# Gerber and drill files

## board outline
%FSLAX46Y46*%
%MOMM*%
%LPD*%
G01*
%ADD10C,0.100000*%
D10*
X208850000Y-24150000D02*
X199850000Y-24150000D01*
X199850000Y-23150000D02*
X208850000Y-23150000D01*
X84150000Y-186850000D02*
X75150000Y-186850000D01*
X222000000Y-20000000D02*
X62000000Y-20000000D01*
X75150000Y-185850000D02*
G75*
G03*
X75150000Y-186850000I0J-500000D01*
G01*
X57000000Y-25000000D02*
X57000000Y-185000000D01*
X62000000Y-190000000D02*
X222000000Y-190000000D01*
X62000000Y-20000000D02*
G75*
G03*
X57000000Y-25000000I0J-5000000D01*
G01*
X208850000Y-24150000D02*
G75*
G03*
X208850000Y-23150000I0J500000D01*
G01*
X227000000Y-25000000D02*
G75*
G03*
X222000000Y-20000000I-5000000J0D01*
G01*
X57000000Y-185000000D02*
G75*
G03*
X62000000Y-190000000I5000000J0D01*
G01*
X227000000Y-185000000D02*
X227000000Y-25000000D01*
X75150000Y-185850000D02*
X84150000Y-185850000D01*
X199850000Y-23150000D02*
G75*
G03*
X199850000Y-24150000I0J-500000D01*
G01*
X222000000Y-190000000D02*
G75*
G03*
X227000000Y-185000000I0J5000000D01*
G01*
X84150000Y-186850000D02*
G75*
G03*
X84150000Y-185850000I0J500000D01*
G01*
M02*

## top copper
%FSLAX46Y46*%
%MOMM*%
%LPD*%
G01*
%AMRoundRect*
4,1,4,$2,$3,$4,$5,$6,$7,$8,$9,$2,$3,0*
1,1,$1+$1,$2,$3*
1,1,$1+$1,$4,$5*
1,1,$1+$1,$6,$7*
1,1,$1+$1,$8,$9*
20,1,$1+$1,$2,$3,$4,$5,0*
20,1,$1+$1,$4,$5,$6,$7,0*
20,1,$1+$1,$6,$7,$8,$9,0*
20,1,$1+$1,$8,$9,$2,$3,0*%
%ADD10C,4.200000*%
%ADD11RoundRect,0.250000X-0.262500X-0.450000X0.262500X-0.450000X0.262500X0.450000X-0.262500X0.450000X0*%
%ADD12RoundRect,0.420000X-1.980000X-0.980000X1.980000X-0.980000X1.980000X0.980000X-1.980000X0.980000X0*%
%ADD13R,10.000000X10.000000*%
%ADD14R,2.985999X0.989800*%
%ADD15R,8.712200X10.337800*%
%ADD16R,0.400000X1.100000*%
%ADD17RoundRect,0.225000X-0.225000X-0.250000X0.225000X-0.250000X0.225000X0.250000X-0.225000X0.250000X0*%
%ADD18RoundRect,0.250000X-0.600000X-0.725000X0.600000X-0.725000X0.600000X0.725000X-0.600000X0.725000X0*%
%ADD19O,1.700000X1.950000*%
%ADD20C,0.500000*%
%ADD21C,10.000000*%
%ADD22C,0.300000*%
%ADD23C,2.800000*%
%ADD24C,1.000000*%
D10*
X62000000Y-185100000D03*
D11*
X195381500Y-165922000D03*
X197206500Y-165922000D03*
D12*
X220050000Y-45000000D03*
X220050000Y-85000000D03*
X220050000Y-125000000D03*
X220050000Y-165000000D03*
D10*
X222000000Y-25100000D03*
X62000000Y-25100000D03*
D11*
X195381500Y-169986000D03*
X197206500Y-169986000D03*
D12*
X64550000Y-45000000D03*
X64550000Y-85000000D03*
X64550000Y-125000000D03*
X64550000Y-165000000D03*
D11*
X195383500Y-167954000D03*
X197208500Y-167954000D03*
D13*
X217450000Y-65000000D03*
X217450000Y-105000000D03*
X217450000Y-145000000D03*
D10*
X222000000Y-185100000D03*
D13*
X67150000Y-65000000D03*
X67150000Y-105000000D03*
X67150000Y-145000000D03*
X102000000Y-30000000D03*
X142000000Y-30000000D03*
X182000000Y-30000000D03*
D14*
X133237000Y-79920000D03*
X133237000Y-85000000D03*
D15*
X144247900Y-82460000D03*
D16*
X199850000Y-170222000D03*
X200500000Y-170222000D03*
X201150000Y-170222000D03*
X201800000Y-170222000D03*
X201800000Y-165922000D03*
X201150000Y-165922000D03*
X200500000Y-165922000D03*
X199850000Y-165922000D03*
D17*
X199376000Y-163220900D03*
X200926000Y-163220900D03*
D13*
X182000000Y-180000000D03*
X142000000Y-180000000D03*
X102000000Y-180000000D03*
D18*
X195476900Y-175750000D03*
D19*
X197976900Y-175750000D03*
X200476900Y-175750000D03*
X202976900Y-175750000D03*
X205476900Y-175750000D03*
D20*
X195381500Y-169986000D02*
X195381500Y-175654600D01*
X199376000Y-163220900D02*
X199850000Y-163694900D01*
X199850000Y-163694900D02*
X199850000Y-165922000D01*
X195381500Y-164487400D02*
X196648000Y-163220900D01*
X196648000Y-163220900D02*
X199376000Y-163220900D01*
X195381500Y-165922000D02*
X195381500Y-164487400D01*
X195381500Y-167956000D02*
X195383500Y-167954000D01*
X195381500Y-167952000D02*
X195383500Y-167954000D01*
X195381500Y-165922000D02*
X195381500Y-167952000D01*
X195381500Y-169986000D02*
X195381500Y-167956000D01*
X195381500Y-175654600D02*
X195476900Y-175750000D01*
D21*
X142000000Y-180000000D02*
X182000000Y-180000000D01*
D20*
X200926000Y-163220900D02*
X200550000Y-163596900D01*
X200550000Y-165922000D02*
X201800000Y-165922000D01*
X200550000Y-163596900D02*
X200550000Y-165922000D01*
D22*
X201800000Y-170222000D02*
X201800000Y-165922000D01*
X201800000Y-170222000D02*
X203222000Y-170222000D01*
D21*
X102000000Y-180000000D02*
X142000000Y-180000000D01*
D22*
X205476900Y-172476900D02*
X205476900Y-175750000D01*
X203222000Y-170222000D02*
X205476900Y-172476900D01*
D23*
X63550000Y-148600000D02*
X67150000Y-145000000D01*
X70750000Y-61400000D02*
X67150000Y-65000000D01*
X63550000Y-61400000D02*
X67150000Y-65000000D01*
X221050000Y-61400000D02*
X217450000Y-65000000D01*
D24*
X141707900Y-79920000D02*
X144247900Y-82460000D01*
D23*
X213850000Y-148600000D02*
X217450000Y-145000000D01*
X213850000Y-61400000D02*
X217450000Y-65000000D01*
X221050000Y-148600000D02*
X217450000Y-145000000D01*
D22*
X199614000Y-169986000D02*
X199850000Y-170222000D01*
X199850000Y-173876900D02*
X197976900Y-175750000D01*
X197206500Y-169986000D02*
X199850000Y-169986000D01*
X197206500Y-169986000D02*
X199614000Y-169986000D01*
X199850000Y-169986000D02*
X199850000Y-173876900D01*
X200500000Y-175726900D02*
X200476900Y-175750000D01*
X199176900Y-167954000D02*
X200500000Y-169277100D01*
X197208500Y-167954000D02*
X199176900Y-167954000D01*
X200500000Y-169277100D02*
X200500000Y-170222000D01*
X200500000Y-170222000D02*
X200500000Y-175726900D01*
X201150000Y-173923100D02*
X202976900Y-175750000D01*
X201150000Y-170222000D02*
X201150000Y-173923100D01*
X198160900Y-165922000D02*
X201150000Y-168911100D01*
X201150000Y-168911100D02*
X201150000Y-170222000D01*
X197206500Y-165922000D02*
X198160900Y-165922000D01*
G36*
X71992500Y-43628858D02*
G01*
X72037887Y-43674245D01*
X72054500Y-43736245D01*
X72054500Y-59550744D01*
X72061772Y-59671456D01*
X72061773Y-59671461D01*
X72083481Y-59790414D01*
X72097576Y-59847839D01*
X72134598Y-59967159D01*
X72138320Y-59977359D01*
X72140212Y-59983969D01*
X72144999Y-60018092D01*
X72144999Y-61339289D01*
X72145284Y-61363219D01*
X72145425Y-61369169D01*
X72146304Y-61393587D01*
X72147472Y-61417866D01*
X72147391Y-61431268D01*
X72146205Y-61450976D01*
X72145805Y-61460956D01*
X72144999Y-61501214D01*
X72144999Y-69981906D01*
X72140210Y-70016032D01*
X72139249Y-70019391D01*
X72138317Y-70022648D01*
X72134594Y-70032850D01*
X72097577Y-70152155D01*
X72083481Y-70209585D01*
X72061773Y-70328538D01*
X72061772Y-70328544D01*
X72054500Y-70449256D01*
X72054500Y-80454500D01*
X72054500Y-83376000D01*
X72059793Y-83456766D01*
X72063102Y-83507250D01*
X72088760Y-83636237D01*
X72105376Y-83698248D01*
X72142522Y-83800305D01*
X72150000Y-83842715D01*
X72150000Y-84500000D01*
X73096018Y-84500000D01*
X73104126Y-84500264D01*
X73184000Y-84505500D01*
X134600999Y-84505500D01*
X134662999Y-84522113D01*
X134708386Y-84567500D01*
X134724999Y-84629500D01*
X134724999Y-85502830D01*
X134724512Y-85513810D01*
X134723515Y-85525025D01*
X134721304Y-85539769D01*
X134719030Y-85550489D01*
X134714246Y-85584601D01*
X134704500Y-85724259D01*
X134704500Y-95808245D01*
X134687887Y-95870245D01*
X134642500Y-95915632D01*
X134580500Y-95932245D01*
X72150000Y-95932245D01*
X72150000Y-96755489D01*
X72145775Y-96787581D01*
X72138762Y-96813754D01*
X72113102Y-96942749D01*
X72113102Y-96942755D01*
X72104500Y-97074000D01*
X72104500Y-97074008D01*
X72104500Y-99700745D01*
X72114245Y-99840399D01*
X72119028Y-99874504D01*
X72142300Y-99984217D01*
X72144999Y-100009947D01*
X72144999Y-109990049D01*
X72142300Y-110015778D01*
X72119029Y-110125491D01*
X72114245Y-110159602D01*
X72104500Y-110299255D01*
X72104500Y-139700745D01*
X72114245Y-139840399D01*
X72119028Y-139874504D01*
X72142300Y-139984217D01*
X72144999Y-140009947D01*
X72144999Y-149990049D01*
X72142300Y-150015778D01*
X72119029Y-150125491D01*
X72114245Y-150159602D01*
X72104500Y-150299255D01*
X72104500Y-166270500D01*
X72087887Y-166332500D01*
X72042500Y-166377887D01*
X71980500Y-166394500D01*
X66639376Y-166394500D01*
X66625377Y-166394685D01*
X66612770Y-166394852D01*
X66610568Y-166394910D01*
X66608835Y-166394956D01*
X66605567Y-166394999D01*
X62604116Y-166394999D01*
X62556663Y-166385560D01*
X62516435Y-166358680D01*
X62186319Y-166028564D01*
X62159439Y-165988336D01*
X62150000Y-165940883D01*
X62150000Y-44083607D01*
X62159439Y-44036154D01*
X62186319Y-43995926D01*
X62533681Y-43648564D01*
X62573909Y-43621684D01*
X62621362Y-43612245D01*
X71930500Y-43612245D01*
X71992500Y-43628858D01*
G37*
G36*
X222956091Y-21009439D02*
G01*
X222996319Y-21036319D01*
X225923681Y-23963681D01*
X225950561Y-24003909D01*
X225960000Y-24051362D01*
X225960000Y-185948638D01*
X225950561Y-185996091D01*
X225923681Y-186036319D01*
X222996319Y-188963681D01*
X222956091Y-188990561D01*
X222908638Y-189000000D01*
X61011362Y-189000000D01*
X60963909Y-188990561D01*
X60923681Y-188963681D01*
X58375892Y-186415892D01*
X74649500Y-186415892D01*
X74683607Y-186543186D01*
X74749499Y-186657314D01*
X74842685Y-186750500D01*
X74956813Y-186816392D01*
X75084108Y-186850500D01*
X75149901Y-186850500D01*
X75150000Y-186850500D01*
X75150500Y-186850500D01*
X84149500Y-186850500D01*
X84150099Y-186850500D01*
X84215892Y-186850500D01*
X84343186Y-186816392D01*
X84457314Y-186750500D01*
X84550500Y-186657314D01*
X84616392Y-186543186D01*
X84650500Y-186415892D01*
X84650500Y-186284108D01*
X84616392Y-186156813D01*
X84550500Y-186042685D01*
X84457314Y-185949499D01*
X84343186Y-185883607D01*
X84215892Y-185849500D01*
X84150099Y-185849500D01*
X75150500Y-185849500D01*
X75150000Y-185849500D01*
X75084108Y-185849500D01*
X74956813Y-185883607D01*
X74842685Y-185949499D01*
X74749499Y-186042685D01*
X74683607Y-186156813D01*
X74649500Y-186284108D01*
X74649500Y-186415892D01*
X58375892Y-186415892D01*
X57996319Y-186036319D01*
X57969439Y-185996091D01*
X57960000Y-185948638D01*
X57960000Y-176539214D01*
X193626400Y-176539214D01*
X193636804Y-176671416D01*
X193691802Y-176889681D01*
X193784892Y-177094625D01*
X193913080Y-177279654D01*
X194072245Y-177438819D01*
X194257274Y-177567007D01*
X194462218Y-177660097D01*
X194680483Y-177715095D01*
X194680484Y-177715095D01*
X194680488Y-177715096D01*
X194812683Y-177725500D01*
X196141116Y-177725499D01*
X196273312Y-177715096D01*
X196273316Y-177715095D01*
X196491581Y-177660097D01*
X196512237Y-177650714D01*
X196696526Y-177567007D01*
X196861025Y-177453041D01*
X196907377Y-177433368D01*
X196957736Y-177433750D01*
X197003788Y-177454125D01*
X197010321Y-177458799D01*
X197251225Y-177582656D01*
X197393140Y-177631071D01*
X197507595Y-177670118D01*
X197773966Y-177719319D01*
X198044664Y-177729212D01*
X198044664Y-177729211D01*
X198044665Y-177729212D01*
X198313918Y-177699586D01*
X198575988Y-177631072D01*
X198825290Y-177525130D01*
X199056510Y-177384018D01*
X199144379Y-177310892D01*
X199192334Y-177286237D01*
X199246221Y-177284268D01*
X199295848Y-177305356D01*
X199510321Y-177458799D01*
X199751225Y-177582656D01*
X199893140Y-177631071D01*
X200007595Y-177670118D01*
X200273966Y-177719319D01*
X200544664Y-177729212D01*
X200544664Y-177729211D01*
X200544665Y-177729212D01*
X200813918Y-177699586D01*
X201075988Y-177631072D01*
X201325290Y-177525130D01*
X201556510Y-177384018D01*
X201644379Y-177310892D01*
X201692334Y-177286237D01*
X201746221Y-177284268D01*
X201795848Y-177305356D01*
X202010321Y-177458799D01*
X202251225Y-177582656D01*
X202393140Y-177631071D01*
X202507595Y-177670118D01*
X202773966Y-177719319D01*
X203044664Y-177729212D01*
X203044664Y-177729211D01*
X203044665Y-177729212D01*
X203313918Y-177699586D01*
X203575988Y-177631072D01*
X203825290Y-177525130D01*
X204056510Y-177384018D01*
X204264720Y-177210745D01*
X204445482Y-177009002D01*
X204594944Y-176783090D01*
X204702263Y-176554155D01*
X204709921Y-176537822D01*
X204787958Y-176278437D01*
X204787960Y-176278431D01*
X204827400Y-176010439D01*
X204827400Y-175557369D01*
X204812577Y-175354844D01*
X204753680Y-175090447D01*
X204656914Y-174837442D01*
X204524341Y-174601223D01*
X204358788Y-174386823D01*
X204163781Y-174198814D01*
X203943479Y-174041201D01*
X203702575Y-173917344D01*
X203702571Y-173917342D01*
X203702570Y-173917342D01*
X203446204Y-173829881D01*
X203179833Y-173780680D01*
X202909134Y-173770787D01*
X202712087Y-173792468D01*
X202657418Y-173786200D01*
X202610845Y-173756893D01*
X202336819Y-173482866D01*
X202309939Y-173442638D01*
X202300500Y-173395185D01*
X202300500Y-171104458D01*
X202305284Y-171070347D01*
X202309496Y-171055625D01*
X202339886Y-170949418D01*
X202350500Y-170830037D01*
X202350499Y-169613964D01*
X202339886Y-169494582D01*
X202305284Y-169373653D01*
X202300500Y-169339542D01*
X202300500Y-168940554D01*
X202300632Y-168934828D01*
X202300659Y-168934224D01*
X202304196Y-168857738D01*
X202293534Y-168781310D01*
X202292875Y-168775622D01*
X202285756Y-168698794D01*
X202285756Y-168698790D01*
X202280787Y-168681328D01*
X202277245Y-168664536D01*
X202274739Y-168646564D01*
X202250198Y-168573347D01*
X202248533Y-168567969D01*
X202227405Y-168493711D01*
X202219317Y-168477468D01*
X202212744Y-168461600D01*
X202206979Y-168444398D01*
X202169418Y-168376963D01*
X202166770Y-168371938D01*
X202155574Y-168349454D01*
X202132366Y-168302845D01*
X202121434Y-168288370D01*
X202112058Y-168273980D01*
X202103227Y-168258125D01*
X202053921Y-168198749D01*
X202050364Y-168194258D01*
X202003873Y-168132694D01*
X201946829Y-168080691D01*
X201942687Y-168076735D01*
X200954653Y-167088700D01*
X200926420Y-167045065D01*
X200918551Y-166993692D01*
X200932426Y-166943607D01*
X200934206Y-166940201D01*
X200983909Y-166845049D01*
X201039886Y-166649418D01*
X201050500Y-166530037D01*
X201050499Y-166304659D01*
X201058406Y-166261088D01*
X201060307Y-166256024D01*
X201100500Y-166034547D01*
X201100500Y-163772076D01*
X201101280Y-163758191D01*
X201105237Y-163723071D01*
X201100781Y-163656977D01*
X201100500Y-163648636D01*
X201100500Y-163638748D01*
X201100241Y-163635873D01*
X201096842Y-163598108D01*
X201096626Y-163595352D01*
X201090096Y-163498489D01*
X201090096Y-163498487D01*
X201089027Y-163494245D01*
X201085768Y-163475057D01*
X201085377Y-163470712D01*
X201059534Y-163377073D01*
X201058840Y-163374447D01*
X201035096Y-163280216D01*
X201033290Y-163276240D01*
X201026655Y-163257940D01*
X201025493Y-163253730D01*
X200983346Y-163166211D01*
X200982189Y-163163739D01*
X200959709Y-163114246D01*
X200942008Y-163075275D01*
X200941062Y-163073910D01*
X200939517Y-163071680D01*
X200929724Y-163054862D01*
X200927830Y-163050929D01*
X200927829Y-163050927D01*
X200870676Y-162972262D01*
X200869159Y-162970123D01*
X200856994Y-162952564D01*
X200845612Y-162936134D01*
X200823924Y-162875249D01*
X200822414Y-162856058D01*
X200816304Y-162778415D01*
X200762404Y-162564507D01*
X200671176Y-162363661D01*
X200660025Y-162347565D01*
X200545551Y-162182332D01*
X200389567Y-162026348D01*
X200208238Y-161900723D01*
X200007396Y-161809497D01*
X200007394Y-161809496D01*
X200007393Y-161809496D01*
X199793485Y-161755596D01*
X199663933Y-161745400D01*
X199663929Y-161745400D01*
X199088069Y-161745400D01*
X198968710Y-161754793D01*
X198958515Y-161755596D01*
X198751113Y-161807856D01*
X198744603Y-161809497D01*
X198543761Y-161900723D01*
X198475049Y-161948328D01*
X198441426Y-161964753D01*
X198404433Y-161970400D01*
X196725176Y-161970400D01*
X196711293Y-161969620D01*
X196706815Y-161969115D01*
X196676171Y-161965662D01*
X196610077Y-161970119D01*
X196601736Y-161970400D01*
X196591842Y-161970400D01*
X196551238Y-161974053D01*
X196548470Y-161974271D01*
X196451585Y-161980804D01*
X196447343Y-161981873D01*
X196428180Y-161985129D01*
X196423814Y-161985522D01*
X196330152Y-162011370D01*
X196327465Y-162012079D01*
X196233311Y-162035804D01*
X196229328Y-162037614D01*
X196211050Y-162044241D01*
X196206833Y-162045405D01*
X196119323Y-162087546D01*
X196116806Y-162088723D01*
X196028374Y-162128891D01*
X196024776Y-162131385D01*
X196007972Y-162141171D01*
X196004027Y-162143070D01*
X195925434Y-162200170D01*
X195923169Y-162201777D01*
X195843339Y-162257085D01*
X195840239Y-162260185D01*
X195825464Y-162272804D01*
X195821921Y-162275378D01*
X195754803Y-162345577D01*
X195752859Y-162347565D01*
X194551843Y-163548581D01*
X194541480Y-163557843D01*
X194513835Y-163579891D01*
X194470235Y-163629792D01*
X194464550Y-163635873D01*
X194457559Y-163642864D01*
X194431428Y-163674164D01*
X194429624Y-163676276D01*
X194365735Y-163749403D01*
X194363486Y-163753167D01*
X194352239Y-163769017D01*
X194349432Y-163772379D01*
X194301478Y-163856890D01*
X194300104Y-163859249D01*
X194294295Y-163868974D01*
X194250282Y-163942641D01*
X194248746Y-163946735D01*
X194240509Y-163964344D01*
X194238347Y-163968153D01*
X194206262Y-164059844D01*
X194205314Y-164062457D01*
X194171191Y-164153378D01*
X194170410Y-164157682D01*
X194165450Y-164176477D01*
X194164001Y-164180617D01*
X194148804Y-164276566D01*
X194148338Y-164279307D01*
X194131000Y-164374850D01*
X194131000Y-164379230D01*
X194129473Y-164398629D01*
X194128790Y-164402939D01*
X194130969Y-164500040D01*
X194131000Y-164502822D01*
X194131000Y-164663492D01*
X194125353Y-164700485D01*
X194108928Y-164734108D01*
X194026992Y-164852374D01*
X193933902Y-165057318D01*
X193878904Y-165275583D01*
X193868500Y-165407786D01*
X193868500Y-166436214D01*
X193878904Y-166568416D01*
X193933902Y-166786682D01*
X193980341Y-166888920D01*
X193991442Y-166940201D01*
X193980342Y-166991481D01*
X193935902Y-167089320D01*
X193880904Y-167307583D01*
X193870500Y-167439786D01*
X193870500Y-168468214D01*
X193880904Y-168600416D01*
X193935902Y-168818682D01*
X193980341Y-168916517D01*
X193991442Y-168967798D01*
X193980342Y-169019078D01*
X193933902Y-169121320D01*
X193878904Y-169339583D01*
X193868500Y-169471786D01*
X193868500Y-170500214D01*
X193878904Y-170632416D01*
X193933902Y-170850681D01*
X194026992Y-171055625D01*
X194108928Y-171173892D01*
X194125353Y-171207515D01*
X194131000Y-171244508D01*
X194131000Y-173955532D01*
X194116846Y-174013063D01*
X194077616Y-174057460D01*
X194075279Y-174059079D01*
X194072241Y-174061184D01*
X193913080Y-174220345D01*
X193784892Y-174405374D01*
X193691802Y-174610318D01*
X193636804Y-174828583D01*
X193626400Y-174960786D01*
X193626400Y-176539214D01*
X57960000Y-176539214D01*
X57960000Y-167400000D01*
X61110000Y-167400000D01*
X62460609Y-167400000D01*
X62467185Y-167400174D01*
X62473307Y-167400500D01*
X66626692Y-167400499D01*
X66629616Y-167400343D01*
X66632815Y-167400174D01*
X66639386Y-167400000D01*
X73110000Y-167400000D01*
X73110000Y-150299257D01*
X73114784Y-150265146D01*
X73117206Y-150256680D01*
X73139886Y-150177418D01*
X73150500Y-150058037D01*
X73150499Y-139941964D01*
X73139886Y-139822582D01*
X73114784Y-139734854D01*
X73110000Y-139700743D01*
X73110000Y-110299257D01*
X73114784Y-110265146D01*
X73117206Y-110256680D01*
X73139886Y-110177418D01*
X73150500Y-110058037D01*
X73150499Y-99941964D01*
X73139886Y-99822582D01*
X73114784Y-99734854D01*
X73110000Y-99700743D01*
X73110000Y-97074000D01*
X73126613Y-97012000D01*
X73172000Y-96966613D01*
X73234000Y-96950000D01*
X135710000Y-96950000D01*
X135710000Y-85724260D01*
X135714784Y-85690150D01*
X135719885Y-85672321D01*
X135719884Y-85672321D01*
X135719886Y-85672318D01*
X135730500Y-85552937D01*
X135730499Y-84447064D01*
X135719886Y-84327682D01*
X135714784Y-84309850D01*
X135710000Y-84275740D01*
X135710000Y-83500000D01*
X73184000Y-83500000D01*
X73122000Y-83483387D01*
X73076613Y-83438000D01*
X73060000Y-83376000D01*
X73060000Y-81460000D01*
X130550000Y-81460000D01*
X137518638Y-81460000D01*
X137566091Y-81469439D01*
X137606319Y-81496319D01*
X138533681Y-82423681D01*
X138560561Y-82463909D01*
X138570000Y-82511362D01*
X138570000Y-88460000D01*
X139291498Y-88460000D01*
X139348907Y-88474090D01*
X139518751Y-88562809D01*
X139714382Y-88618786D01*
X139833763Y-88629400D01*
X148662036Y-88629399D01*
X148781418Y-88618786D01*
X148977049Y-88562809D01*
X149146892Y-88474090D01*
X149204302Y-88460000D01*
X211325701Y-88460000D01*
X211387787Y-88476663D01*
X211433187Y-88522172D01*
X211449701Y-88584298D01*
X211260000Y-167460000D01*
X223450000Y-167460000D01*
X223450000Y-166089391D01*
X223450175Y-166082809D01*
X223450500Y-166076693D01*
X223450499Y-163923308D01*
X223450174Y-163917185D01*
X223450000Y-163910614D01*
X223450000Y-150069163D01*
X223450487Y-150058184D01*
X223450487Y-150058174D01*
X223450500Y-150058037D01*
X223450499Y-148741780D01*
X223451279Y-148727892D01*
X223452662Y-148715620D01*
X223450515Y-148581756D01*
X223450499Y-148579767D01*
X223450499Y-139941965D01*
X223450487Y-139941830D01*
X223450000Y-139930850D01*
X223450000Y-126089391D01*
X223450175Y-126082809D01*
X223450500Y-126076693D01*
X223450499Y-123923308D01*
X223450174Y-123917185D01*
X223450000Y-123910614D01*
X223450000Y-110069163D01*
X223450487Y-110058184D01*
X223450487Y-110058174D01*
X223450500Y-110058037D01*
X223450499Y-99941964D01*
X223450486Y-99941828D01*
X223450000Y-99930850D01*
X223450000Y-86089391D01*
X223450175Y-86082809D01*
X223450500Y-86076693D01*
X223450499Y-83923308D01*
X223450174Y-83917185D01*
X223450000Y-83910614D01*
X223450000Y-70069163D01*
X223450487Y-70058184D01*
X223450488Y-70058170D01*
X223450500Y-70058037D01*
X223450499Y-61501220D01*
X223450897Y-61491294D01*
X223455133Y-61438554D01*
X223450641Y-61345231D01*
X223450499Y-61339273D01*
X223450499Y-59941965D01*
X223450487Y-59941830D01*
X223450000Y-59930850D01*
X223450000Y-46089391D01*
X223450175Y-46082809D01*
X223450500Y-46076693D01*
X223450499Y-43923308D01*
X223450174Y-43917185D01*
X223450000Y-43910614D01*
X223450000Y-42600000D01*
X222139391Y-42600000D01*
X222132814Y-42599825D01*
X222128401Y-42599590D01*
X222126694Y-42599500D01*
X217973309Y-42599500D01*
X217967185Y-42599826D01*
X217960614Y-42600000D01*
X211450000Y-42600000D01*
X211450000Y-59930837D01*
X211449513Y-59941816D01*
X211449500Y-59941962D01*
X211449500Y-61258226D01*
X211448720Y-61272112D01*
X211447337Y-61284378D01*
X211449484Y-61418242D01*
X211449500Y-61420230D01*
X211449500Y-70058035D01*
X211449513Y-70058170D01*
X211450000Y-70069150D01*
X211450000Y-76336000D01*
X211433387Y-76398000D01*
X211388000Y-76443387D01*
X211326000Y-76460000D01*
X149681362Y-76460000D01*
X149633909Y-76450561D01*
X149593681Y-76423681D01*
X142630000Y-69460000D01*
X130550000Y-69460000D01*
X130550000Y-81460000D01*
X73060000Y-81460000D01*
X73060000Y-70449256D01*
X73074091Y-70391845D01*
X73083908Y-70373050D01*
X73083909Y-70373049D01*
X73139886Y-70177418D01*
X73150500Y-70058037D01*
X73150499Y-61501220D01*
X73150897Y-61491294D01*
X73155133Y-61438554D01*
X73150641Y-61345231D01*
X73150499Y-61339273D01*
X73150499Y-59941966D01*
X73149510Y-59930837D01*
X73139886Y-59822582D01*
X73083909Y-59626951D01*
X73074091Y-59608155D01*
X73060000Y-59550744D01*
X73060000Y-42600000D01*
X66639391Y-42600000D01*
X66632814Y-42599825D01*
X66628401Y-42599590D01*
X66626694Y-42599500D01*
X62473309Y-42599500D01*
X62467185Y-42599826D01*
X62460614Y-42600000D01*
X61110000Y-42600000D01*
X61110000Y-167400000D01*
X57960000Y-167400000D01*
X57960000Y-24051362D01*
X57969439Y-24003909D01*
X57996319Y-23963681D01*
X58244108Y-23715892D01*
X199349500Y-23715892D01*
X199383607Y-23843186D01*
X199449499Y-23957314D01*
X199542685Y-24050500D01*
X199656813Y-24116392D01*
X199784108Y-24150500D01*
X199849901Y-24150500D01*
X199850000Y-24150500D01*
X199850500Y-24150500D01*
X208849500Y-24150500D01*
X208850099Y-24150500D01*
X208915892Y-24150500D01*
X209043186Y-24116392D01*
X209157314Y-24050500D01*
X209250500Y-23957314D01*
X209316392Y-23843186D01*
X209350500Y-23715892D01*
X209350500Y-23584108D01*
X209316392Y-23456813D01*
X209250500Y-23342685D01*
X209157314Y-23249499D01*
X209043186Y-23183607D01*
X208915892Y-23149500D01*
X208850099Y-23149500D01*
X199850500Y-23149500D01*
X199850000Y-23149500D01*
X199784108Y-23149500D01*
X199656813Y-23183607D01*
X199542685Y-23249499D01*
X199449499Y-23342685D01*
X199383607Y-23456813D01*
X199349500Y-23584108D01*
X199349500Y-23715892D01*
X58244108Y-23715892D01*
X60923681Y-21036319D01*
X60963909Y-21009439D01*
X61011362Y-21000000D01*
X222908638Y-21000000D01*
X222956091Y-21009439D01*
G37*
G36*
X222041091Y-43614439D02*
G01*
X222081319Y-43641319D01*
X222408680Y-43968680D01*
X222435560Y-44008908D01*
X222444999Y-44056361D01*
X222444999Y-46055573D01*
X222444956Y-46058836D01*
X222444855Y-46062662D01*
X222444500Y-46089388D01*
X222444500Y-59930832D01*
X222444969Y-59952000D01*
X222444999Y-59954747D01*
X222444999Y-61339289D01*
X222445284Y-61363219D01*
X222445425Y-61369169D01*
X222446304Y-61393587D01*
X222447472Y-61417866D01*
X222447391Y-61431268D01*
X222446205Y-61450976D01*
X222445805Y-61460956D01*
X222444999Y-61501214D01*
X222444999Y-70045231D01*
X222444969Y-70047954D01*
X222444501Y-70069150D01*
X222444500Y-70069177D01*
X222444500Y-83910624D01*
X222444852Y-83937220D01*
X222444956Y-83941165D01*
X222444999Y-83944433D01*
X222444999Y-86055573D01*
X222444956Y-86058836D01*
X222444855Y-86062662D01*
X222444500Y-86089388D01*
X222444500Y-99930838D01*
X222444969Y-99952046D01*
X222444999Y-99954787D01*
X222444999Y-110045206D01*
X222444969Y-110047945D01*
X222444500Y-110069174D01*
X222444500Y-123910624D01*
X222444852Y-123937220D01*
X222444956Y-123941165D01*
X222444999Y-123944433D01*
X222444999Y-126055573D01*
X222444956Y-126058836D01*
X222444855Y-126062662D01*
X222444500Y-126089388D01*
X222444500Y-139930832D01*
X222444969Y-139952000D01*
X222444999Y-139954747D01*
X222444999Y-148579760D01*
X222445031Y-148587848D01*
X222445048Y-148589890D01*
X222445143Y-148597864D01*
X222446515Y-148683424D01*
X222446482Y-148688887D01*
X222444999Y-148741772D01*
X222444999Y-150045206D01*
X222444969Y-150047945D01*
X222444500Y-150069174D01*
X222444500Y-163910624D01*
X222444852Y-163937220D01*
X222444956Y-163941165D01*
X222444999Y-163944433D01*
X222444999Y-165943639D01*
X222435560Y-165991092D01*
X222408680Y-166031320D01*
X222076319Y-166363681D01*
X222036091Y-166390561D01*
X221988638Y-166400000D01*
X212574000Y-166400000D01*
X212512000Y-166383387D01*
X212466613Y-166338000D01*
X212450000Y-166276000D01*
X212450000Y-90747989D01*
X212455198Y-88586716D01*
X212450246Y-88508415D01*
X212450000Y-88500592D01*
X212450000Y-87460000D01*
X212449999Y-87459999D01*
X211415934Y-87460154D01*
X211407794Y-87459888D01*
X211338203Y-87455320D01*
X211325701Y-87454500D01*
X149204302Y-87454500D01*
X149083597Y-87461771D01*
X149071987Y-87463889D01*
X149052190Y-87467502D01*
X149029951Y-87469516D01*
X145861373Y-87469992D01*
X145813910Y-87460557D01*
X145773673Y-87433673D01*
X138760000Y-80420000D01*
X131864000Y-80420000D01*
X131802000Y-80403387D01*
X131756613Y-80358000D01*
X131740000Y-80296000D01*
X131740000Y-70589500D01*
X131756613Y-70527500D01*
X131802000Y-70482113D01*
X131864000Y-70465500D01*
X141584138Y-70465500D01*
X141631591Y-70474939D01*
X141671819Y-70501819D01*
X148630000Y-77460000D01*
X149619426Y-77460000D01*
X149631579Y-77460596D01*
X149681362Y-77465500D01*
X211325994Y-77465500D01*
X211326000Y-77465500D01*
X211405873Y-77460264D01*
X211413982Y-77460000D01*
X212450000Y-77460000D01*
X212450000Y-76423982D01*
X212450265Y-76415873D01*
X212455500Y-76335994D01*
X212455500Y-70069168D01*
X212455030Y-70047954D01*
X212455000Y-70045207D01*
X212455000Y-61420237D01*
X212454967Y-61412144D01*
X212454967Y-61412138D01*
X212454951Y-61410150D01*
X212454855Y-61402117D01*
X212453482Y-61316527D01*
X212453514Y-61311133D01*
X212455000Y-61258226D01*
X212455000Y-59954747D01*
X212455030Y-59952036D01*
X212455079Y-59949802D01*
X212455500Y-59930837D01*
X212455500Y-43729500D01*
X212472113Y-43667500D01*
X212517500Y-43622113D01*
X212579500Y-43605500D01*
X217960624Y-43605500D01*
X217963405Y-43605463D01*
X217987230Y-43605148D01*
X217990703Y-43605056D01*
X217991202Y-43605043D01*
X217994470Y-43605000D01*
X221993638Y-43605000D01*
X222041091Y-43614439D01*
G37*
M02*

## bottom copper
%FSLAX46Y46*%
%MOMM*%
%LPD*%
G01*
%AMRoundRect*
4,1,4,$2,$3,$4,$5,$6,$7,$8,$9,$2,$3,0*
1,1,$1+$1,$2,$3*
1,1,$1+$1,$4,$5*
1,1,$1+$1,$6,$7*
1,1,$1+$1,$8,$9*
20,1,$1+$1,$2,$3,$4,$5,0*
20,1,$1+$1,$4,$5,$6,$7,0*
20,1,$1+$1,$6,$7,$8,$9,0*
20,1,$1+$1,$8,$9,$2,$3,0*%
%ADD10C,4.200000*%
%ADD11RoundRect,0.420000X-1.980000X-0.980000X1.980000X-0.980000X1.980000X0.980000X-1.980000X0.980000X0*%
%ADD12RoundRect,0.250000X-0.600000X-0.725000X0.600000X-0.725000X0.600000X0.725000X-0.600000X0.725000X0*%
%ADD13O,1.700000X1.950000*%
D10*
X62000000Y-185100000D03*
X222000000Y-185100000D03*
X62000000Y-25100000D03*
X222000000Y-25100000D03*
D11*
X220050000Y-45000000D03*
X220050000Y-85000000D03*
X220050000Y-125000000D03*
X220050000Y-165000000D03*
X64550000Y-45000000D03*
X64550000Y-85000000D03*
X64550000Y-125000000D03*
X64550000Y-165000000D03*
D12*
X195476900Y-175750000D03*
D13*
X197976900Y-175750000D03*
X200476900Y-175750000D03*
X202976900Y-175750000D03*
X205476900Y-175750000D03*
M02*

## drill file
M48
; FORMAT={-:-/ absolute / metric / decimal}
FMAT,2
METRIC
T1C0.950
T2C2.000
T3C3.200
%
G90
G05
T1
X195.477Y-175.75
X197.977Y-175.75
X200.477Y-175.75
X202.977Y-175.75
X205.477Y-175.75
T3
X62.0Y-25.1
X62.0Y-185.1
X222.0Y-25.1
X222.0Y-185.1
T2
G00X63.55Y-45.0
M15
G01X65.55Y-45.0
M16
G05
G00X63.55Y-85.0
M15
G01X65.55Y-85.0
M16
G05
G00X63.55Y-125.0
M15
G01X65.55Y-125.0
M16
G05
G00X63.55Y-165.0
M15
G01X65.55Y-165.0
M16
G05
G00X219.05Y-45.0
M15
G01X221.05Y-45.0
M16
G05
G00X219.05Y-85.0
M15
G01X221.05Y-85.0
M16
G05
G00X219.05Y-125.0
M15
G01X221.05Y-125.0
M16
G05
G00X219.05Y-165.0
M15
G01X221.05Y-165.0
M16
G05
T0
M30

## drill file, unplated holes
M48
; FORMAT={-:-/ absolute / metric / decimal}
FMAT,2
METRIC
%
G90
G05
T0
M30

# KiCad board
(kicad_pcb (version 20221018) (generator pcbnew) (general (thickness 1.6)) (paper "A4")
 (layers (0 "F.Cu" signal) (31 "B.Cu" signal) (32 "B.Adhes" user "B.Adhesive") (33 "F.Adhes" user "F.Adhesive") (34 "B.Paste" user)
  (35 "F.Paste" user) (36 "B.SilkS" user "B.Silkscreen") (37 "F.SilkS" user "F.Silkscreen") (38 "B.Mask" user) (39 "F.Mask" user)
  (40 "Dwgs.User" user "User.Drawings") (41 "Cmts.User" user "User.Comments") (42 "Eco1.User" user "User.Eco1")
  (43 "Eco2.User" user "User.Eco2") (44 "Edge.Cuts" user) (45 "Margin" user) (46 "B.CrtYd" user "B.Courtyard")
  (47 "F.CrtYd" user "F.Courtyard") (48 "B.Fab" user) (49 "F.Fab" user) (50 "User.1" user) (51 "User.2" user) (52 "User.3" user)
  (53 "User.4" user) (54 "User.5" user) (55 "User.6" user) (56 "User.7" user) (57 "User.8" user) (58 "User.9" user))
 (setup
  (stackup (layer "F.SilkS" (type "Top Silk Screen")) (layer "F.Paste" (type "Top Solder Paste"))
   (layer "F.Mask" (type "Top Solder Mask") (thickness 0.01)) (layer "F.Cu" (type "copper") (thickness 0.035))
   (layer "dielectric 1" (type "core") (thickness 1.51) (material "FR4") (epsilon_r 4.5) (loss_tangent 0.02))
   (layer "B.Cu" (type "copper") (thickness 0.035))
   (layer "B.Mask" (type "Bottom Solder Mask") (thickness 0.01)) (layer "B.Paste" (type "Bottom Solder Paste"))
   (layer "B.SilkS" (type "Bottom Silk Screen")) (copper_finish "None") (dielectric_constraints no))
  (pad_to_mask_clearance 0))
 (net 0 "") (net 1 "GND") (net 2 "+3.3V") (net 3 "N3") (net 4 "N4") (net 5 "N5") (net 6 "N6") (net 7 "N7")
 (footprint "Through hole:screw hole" (layer "F.Cu") (at 62 185)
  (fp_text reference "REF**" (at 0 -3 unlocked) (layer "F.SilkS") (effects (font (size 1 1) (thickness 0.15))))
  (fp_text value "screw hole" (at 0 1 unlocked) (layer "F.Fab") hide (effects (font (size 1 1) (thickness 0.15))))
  (pad "1" thru_hole circle (at 0 0.1) (size 4.2 4.2) (drill 3.2) (layers "*.Cu" "*.Mask") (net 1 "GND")))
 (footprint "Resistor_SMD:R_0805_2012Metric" (layer "F.Cu") (at 196.294 165.922)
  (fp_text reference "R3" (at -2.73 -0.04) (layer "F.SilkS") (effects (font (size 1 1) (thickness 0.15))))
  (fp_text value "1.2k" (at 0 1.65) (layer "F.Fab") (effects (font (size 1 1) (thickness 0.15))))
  (pad "1" smd roundrect (at -0.9125 0) (size 1.025 1.4) (layers "F.Cu" "F.Paste" "F.Mask") (roundrect_rratio 0.243902439) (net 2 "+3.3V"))
  (pad "2" smd roundrect (at 0.9125 0) (size 1.025 1.4) (layers "F.Cu" "F.Paste" "F.Mask") (roundrect_rratio 0.243902439) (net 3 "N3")))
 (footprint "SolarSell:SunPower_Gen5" (layer "F.Cu") (at 220.05 45)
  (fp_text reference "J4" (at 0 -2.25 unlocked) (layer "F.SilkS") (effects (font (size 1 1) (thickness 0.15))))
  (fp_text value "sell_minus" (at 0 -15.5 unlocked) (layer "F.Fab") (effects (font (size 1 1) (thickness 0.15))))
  (pad "1" thru_hole roundrect (at 0 0) (size 4.8 2.8) (drill oval 4 2) (layers "*.Cu" "*.Mask") (roundrect_rratio 0.15) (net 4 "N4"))
  (pad "2" thru_hole roundrect (at 0 40) (size 4.8 2.8) (drill oval 4 2) (layers "*.Cu" "*.Mask") (roundrect_rratio 0.15) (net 4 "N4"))
  (pad "3" thru_hole roundrect (at 0 80) (size 4.8 2.8) (drill oval 4 2) (layers "*.Cu" "*.Mask") (roundrect_rratio 0.15) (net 4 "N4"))
  (pad "4" thru_hole roundrect (at 0 120) (size 4.8 2.8) (drill oval 4 2) (layers "*.Cu" "*.Mask") (roundrect_rratio 0.15) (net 4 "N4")))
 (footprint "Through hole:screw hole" (layer "F.Cu") (at 222 25)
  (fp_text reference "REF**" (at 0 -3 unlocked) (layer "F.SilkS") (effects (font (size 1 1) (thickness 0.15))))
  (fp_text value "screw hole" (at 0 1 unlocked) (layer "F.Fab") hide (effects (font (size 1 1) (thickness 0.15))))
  (pad "1" thru_hole circle (at 0 0.1) (size 4.2 4.2) (drill 3.2) (layers "*.Cu" "*.Mask") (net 1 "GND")))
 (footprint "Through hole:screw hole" (layer "F.Cu") (at 62 25)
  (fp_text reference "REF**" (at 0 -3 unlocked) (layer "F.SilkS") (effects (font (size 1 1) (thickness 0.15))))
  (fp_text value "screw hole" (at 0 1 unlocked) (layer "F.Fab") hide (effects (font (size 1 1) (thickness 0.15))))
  (pad "1" thru_hole circle (at 0 0.1) (size 4.2 4.2) (drill 3.2) (layers "*.Cu" "*.Mask") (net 1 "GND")))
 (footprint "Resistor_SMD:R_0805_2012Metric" (layer "F.Cu") (at 196.294 169.986)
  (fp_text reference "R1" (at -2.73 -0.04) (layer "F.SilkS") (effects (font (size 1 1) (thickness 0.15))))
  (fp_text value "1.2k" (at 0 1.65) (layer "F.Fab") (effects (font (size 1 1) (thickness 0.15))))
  (pad "1" smd roundrect (at -0.9125 0) (size 1.025 1.4) (layers "F.Cu" "F.Paste" "F.Mask") (roundrect_rratio 0.243902439) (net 2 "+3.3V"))
  (pad "2" smd roundrect (at 0.9125 0) (size 1.025 1.4) (layers "F.Cu" "F.Paste" "F.Mask") (roundrect_rratio 0.243902439) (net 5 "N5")))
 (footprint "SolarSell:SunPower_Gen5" (layer "F.Cu") (at 64.55 45)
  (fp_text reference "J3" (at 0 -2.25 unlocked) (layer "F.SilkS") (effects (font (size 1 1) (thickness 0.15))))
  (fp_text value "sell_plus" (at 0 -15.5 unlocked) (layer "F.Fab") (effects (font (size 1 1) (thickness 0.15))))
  (pad "1" thru_hole roundrect (at 0 0) (size 4.8 2.8) (drill oval 4 2) (layers "*.Cu" "*.Mask") (roundrect_rratio 0.15) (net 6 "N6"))
  (pad "2" thru_hole roundrect (at 0 40) (size 4.8 2.8) (drill oval 4 2) (layers "*.Cu" "*.Mask") (roundrect_rratio 0.15) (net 6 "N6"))
  (pad "3" thru_hole roundrect (at 0 80) (size 4.8 2.8) (drill oval 4 2) (layers "*.Cu" "*.Mask") (roundrect_rratio 0.15) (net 6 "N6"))
  (pad "4" thru_hole roundrect (at 0 120) (size 4.8 2.8) (drill oval 4 2) (layers "*.Cu" "*.Mask") (roundrect_rratio 0.15) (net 6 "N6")))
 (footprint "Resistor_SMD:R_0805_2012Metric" (layer "F.Cu") (at 196.296 167.954)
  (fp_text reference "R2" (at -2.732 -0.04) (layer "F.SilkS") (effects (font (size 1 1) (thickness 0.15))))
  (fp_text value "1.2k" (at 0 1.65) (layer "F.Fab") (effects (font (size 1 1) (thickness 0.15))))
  (pad "1" smd roundrect (at -0.9125 0) (size 1.025 1.4) (layers "F.Cu" "F.Paste" "F.Mask") (roundrect_rratio 0.243902439) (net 2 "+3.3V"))
  (pad "2" smd roundrect (at 0.9125 0) (size 1.025 1.4) (layers "F.Cu" "F.Paste" "F.Mask") (roundrect_rratio 0.243902439) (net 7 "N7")))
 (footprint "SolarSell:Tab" (layer "F.Cu") (at 217.45 105)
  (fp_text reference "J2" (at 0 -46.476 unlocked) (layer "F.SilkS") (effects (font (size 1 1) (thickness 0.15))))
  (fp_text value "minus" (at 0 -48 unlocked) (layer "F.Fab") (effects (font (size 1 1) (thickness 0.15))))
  (pad "1" smd rect (at 0 -40) (size 10 10) (layers "F.Cu" "F.Paste" "F.Mask") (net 4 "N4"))
  (pad "2" smd rect (at 0 0) (size 10 10) (layers "F.Cu" "F.Paste" "F.Mask") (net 4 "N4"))
  (pad "3" smd rect (at 0 40) (size 10 10) (layers "F.Cu" "F.Paste" "F.Mask") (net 4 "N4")))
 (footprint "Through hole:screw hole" (layer "F.Cu") (at 222 185)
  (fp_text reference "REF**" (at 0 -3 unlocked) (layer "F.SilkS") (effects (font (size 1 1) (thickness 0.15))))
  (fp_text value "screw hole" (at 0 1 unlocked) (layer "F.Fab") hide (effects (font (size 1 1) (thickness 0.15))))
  (pad "1" thru_hole circle (at 0 0.1) (size 4.2 4.2) (drill 3.2) (layers "*.Cu" "*.Mask") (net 1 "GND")))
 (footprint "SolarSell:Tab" (layer "F.Cu") (at 67.15 105)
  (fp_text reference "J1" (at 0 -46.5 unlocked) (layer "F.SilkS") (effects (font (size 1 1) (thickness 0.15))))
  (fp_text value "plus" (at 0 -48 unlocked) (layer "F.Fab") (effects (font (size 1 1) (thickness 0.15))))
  (pad "1" smd rect (at 0 -40) (size 10 10) (layers "F.Cu" "F.Paste" "F.Mask") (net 6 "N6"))
  (pad "2" smd rect (at 0 0) (size 10 10) (layers "F.Cu" "F.Paste" "F.Mask") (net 6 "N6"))
  (pad "3" smd rect (at 0 40) (size 10 10) (layers "F.Cu" "F.Paste" "F.Mask") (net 6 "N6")))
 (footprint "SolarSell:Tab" (layer "F.Cu") (at 142 30 90)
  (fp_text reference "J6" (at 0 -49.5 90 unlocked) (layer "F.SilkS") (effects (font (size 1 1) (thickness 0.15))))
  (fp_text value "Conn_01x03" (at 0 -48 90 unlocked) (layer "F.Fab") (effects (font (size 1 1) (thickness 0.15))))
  (pad "1" smd rect (at 0 -40 90) (size 10 10) (layers "F.Cu" "F.Paste" "F.Mask") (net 1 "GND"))
  (pad "2" smd rect (at 0 0 90) (size 10 10) (layers "F.Cu" "F.Paste" "F.Mask") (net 1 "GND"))
  (pad "3" smd rect (at 0 40 90) (size 10 10) (layers "F.Cu" "F.Paste" "F.Mask") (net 1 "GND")))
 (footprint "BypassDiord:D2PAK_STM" (layer "F.Cu") (at 142 82.46 -90)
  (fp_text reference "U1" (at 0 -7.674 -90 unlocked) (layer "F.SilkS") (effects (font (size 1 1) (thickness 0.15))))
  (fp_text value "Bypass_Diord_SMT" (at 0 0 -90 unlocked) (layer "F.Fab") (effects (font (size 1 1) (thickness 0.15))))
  (pad "1" smd rect (at -2.54 8.763 270) (size 0.9898 2.985999) (layers "F.Cu" "F.Paste" "F.Mask") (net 4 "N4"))
  (pad "2" smd rect (at 2.54 8.763 270) (size 0.9898 2.985999) (layers "F.Cu" "F.Paste" "F.Mask") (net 6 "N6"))
  (pad "3" smd rect (at 0 -2.2479 270) (size 10.3378 8.7122) (layers "F.Cu" "F.Paste" "F.Mask") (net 4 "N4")))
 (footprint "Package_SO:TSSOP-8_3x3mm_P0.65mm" (layer "F.Cu") (at 200.825 168.072 90)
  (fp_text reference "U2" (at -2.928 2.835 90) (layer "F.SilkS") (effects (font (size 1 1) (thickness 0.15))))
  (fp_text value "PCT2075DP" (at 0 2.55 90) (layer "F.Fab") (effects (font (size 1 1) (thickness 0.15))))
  (pad "1" smd rect (at -2.15 -0.975 90) (size 1.1 0.4) (layers "F.Cu" "F.Paste" "F.Mask") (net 5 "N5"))
  (pad "2" smd rect (at -2.15 -0.325 90) (size 1.1 0.4) (layers "F.Cu" "F.Paste" "F.Mask") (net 7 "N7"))
  (pad "3" smd rect (at -2.15 0.325 90) (size 1.1 0.4) (layers "F.Cu" "F.Paste" "F.Mask") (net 3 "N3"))
  (pad "4" smd rect (at -2.15 0.975 90) (size 1.1 0.4) (layers "F.Cu" "F.Paste" "F.Mask") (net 1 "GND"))
  (pad "5" smd rect (at 2.15 0.975 90) (size 1.1 0.4) (layers "F.Cu" "F.Paste" "F.Mask") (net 1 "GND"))
  (pad "6" smd rect (at 2.15 0.325 90) (size 1.1 0.4) (layers "F.Cu" "F.Paste" "F.Mask") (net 1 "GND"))
  (pad "7" smd rect (at 2.15 -0.325 90) (size 1.1 0.4) (layers "F.Cu" "F.Paste" "F.Mask") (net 1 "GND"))
  (pad "8" smd rect (at 2.15 -0.975 90) (size 1.1 0.4) (layers "F.Cu" "F.Paste" "F.Mask") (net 2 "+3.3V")))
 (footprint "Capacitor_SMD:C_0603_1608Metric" (layer "F.Cu") (at 200.151 163.2209)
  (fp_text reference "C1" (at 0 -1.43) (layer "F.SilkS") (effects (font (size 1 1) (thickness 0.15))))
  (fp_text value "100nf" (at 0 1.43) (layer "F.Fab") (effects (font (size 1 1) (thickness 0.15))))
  (pad "1" smd roundrect (at -0.775 0) (size 0.9 0.95) (layers "F.Cu" "F.Paste" "F.Mask") (roundrect_rratio 0.25) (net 2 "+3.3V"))
  (pad "2" smd roundrect (at 0.775 0) (size 0.9 0.95) (layers "F.Cu" "F.Paste" "F.Mask") (roundrect_rratio 0.25) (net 1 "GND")))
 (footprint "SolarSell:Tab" (layer "F.Cu") (at 142 180 -90)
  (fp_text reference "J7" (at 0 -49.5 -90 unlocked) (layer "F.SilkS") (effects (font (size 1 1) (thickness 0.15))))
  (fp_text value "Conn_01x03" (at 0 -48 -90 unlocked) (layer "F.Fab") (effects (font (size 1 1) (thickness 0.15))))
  (pad "1" smd rect (at 0 -40 270) (size 10 10) (layers "F.Cu" "F.Paste" "F.Mask") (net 1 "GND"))
  (pad "2" smd rect (at 0 0 270) (size 10 10) (layers "F.Cu" "F.Paste" "F.Mask") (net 1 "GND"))
  (pad "3" smd rect (at 0 40 270) (size 10 10) (layers "F.Cu" "F.Paste" "F.Mask") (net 1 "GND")))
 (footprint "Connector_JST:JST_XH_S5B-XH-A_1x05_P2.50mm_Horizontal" (layer "F.Cu") (at 195.4769 175.75)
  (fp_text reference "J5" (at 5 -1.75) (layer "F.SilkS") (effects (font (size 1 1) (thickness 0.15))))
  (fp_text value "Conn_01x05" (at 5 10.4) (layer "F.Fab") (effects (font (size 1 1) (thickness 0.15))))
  (pad "1" thru_hole roundrect (at 0 0) (size 1.7 1.95) (drill 0.95) (layers "*.Cu" "*.Mask") (roundrect_rratio 0.1470588235)
   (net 2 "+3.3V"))
  (pad "2" thru_hole oval (at 2.5 0) (size 1.7 1.95) (drill 0.95) (layers "*.Cu" "*.Mask") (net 5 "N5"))
  (pad "3" thru_hole oval (at 5 0) (size 1.7 1.95) (drill 0.95) (layers "*.Cu" "*.Mask") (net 7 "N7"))
  (pad "4" thru_hole oval (at 7.5 0) (size 1.7 1.95) (drill 0.95) (layers "*.Cu" "*.Mask") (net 3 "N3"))
  (pad "5" thru_hole oval (at 10 0) (size 1.7 1.95) (drill 0.95) (layers "*.Cu" "*.Mask") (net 1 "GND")))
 (gr_line (start 208.85 24.15) (end 199.85 24.15) (stroke (width 0.1) (type default)) (layer "Edge.Cuts"))
 (gr_line (start 199.85 23.15) (end 208.85 23.15) (stroke (width 0.1) (type default)) (layer "Edge.Cuts"))
 (gr_line (start 84.15 186.85) (end 75.15 186.85) (stroke (width 0.1) (type default)) (layer "Edge.Cuts"))
 (gr_line (start 222 20) (end 62 20) (stroke (width 0.1) (type default)) (layer "Edge.Cuts"))
 (gr_arc (start 75.15 186.85) (mid 74.65 186.35) (end 75.15 185.85) (stroke (width 0.1) (type default)) (layer "Edge.Cuts"))
 (gr_line (start 57 25) (end 57 185) (stroke (width 0.1) (type default)) (layer "Edge.Cuts"))
 (gr_line (start 62 190) (end 222 190) (stroke (width 0.1) (type default)) (layer "Edge.Cuts"))
 (gr_arc (start 57 25) (mid 58.464466 21.464466) (end 62 20) (stroke (width 0.1) (type default)) (layer "Edge.Cuts"))
 (gr_arc (start 208.85 23.15) (mid 209.35 23.65) (end 208.85 24.15) (stroke (width 0.1) (type default)) (layer "Edge.Cuts"))
 (gr_arc (start 222 20) (mid 225.535534 21.464466) (end 227 25) (stroke (width 0.1) (type default)) (layer "Edge.Cuts"))
 (gr_arc (start 62 190) (mid 58.464466 188.535534) (end 57 185) (stroke (width 0.1) (type default)) (layer "Edge.Cuts"))
 (gr_line (start 227 185) (end 227 25) (stroke (width 0.1) (type default)) (layer "Edge.Cuts"))
 (gr_line (start 75.15 185.85) (end 84.15 185.85) (stroke (width 0.1) (type default)) (layer "Edge.Cuts"))
 (gr_arc (start 199.85 24.15) (mid 199.35 23.65) (end 199.85 23.15) (stroke (width 0.1) (type default)) (layer "Edge.Cuts"))
 (gr_arc (start 227 185) (mid 225.535534 188.535534) (end 222 190) (stroke (width 0.1) (type default)) (layer "Edge.Cuts"))
 (gr_arc (start 84.15 185.85) (mid 84.65 186.35) (end 84.15 186.85) (stroke (width 0.1) (type default)) (layer "Edge.Cuts"))
 (segment (start 195.3815 169.986) (end 195.3815 175.6546) (width 0.5) (layer "F.Cu") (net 2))
 (segment (start 199.376 163.2209) (end 199.85 163.6949) (width 0.5) (layer "F.Cu") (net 2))
 (segment (start 199.85 163.6949) (end 199.85 165.922) (width 0.5) (layer "F.Cu") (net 2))
 (segment (start 195.3815 164.4874) (end 196.648 163.2209) (width 0.5) (layer "F.Cu") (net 2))
 (segment (start 196.648 163.2209) (end 199.376 163.2209) (width 0.5) (layer "F.Cu") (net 2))
 (segment (start 195.3815 165.922) (end 195.3815 164.4874) (width 0.5) (layer "F.Cu") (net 2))
 (segment (start 195.3815 167.956) (end 195.3835 167.954) (width 0.5) (layer "F.Cu") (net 2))
 (segment (start 195.3815 167.952) (end 195.3835 167.954) (width 0.5) (layer "F.Cu") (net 2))
 (segment (start 195.3815 165.922) (end 195.3815 167.952) (width 0.5) (layer "F.Cu") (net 2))
 (segment (start 195.3815 169.986) (end 195.3815 167.956) (width 0.5) (layer "F.Cu") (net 2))
 (segment (start 195.3815 175.6546) (end 195.4769 175.75) (width 0.5) (layer "F.Cu") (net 2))
 (segment (start 142 180) (end 182 180) (width 10) (layer "F.Cu") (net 1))
 (segment (start 200.926 163.2209) (end 200.55 163.5969) (width 0.5) (layer "F.Cu") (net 1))
 (segment (start 200.55 165.922) (end 201.8 165.922) (width 0.5) (layer "F.Cu") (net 1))
 (segment (start 200.55 163.5969) (end 200.55 165.922) (width 0.5) (layer "F.Cu") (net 1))
 (segment (start 201.8 170.222) (end 201.8 165.922) (width 0.3) (layer "F.Cu") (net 1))
 (segment (start 201.8 170.222) (end 203.222 170.222) (width 0.3) (layer "F.Cu") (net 1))
 (segment (start 102 180) (end 142 180) (width 10) (layer "F.Cu") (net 1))
 (segment (start 205.4769 172.4769) (end 205.4769 175.75) (width 0.3) (layer "F.Cu") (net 1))
 (segment (start 203.222 170.222) (end 205.4769 172.4769) (width 0.3) (layer "F.Cu") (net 1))
 (segment (start 63.55 148.6) (end 67.15 145) (width 2.8) (layer "F.Cu") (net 6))
 (segment (start 70.75 61.4) (end 67.15 65) (width 2.8) (layer "F.Cu") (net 6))
 (segment (start 63.55 61.4) (end 67.15 65) (width 2.8) (layer "F.Cu") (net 6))
 (segment (start 221.05 61.4) (end 217.45 65) (width 2.8) (layer "F.Cu") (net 4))
 (segment (start 141.7079 79.92) (end 144.2479 82.46) (width 1) (layer "F.Cu") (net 4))
 (segment (start 213.85 148.6) (end 217.45 145) (width 2.8) (layer "F.Cu") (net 4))
 (segment (start 213.85 61.4) (end 217.45 65) (width 2.8) (layer "F.Cu") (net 4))
 (segment (start 221.05 148.6) (end 217.45 145) (width 2.8) (layer "F.Cu") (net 4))
 (segment (start 199.614 169.986) (end 199.85 170.222) (width 0.3) (layer "F.Cu") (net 5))
 (segment (start 199.85 173.8769) (end 197.9769 175.75) (width 0.3) (layer "F.Cu") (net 5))
 (segment (start 197.2065 169.986) (end 199.85 169.986) (width 0.3) (layer "F.Cu") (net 5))
 (segment (start 197.2065 169.986) (end 199.614 169.986) (width 0.3) (layer "F.Cu") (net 5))
 (segment (start 199.85 169.986) (end 199.85 173.8769) (width 0.3) (layer "F.Cu") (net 5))
 (segment (start 200.5 175.7269) (end 200.4769 175.75) (width 0.3) (layer "F.Cu") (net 7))
 (segment (start 199.1769 167.954) (end 200.5 169.2771) (width 0.3) (layer "F.Cu") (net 7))
 (segment (start 197.2085 167.954) (end 199.1769 167.954) (width 0.3) (layer "F.Cu") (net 7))
 (segment (start 200.5 169.2771) (end 200.5 170.222) (width 0.3) (layer "F.Cu") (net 7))
 (segment (start 200.5 170.222) (end 200.5 175.7269) (width 0.3) (layer "F.Cu") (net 7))
 (segment (start 201.15 173.9231) (end 202.9769 175.75) (width 0.3) (layer "F.Cu") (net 3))
 (segment (start 201.15 170.222) (end 201.15 173.9231) (width 0.3) (layer "F.Cu") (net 3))
 (segment (start 198.1609 165.922) (end 201.15 168.9111) (width 0.3) (layer "F.Cu") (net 3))
 (segment (start 201.15 168.9111) (end 201.15 170.222) (width 0.3) (layer "F.Cu") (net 3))
 (segment (start 197.2065 165.922) (end 198.1609 165.922) (width 0.3) (layer "F.Cu") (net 3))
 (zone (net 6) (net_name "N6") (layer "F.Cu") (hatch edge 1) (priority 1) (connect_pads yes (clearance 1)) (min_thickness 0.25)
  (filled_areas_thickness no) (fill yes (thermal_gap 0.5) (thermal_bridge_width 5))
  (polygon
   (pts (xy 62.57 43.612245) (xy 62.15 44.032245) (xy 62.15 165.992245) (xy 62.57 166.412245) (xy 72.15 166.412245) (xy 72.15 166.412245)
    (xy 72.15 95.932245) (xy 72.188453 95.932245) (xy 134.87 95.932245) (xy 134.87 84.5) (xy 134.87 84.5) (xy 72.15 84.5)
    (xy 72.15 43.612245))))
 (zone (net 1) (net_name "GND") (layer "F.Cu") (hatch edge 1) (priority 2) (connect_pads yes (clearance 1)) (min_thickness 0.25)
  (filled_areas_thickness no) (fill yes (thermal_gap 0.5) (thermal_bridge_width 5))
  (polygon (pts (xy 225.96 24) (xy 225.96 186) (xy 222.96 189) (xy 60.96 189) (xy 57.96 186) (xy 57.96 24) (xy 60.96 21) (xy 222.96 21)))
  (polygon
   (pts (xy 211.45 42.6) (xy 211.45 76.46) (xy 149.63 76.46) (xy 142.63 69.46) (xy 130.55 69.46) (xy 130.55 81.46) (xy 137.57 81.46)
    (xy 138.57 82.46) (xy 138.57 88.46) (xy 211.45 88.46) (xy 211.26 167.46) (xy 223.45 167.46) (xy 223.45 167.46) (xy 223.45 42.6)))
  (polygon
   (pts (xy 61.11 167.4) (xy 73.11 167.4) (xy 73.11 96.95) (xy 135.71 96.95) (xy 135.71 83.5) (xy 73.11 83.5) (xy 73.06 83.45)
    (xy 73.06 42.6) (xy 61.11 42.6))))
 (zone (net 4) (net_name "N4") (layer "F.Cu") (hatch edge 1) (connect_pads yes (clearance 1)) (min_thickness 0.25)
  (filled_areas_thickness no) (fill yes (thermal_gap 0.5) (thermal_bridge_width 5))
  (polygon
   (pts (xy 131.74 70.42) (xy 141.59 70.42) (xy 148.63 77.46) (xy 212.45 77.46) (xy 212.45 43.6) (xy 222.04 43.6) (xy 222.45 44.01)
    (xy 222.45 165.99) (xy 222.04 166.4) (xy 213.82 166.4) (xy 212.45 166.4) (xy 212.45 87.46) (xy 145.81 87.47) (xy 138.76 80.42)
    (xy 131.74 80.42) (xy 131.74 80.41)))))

